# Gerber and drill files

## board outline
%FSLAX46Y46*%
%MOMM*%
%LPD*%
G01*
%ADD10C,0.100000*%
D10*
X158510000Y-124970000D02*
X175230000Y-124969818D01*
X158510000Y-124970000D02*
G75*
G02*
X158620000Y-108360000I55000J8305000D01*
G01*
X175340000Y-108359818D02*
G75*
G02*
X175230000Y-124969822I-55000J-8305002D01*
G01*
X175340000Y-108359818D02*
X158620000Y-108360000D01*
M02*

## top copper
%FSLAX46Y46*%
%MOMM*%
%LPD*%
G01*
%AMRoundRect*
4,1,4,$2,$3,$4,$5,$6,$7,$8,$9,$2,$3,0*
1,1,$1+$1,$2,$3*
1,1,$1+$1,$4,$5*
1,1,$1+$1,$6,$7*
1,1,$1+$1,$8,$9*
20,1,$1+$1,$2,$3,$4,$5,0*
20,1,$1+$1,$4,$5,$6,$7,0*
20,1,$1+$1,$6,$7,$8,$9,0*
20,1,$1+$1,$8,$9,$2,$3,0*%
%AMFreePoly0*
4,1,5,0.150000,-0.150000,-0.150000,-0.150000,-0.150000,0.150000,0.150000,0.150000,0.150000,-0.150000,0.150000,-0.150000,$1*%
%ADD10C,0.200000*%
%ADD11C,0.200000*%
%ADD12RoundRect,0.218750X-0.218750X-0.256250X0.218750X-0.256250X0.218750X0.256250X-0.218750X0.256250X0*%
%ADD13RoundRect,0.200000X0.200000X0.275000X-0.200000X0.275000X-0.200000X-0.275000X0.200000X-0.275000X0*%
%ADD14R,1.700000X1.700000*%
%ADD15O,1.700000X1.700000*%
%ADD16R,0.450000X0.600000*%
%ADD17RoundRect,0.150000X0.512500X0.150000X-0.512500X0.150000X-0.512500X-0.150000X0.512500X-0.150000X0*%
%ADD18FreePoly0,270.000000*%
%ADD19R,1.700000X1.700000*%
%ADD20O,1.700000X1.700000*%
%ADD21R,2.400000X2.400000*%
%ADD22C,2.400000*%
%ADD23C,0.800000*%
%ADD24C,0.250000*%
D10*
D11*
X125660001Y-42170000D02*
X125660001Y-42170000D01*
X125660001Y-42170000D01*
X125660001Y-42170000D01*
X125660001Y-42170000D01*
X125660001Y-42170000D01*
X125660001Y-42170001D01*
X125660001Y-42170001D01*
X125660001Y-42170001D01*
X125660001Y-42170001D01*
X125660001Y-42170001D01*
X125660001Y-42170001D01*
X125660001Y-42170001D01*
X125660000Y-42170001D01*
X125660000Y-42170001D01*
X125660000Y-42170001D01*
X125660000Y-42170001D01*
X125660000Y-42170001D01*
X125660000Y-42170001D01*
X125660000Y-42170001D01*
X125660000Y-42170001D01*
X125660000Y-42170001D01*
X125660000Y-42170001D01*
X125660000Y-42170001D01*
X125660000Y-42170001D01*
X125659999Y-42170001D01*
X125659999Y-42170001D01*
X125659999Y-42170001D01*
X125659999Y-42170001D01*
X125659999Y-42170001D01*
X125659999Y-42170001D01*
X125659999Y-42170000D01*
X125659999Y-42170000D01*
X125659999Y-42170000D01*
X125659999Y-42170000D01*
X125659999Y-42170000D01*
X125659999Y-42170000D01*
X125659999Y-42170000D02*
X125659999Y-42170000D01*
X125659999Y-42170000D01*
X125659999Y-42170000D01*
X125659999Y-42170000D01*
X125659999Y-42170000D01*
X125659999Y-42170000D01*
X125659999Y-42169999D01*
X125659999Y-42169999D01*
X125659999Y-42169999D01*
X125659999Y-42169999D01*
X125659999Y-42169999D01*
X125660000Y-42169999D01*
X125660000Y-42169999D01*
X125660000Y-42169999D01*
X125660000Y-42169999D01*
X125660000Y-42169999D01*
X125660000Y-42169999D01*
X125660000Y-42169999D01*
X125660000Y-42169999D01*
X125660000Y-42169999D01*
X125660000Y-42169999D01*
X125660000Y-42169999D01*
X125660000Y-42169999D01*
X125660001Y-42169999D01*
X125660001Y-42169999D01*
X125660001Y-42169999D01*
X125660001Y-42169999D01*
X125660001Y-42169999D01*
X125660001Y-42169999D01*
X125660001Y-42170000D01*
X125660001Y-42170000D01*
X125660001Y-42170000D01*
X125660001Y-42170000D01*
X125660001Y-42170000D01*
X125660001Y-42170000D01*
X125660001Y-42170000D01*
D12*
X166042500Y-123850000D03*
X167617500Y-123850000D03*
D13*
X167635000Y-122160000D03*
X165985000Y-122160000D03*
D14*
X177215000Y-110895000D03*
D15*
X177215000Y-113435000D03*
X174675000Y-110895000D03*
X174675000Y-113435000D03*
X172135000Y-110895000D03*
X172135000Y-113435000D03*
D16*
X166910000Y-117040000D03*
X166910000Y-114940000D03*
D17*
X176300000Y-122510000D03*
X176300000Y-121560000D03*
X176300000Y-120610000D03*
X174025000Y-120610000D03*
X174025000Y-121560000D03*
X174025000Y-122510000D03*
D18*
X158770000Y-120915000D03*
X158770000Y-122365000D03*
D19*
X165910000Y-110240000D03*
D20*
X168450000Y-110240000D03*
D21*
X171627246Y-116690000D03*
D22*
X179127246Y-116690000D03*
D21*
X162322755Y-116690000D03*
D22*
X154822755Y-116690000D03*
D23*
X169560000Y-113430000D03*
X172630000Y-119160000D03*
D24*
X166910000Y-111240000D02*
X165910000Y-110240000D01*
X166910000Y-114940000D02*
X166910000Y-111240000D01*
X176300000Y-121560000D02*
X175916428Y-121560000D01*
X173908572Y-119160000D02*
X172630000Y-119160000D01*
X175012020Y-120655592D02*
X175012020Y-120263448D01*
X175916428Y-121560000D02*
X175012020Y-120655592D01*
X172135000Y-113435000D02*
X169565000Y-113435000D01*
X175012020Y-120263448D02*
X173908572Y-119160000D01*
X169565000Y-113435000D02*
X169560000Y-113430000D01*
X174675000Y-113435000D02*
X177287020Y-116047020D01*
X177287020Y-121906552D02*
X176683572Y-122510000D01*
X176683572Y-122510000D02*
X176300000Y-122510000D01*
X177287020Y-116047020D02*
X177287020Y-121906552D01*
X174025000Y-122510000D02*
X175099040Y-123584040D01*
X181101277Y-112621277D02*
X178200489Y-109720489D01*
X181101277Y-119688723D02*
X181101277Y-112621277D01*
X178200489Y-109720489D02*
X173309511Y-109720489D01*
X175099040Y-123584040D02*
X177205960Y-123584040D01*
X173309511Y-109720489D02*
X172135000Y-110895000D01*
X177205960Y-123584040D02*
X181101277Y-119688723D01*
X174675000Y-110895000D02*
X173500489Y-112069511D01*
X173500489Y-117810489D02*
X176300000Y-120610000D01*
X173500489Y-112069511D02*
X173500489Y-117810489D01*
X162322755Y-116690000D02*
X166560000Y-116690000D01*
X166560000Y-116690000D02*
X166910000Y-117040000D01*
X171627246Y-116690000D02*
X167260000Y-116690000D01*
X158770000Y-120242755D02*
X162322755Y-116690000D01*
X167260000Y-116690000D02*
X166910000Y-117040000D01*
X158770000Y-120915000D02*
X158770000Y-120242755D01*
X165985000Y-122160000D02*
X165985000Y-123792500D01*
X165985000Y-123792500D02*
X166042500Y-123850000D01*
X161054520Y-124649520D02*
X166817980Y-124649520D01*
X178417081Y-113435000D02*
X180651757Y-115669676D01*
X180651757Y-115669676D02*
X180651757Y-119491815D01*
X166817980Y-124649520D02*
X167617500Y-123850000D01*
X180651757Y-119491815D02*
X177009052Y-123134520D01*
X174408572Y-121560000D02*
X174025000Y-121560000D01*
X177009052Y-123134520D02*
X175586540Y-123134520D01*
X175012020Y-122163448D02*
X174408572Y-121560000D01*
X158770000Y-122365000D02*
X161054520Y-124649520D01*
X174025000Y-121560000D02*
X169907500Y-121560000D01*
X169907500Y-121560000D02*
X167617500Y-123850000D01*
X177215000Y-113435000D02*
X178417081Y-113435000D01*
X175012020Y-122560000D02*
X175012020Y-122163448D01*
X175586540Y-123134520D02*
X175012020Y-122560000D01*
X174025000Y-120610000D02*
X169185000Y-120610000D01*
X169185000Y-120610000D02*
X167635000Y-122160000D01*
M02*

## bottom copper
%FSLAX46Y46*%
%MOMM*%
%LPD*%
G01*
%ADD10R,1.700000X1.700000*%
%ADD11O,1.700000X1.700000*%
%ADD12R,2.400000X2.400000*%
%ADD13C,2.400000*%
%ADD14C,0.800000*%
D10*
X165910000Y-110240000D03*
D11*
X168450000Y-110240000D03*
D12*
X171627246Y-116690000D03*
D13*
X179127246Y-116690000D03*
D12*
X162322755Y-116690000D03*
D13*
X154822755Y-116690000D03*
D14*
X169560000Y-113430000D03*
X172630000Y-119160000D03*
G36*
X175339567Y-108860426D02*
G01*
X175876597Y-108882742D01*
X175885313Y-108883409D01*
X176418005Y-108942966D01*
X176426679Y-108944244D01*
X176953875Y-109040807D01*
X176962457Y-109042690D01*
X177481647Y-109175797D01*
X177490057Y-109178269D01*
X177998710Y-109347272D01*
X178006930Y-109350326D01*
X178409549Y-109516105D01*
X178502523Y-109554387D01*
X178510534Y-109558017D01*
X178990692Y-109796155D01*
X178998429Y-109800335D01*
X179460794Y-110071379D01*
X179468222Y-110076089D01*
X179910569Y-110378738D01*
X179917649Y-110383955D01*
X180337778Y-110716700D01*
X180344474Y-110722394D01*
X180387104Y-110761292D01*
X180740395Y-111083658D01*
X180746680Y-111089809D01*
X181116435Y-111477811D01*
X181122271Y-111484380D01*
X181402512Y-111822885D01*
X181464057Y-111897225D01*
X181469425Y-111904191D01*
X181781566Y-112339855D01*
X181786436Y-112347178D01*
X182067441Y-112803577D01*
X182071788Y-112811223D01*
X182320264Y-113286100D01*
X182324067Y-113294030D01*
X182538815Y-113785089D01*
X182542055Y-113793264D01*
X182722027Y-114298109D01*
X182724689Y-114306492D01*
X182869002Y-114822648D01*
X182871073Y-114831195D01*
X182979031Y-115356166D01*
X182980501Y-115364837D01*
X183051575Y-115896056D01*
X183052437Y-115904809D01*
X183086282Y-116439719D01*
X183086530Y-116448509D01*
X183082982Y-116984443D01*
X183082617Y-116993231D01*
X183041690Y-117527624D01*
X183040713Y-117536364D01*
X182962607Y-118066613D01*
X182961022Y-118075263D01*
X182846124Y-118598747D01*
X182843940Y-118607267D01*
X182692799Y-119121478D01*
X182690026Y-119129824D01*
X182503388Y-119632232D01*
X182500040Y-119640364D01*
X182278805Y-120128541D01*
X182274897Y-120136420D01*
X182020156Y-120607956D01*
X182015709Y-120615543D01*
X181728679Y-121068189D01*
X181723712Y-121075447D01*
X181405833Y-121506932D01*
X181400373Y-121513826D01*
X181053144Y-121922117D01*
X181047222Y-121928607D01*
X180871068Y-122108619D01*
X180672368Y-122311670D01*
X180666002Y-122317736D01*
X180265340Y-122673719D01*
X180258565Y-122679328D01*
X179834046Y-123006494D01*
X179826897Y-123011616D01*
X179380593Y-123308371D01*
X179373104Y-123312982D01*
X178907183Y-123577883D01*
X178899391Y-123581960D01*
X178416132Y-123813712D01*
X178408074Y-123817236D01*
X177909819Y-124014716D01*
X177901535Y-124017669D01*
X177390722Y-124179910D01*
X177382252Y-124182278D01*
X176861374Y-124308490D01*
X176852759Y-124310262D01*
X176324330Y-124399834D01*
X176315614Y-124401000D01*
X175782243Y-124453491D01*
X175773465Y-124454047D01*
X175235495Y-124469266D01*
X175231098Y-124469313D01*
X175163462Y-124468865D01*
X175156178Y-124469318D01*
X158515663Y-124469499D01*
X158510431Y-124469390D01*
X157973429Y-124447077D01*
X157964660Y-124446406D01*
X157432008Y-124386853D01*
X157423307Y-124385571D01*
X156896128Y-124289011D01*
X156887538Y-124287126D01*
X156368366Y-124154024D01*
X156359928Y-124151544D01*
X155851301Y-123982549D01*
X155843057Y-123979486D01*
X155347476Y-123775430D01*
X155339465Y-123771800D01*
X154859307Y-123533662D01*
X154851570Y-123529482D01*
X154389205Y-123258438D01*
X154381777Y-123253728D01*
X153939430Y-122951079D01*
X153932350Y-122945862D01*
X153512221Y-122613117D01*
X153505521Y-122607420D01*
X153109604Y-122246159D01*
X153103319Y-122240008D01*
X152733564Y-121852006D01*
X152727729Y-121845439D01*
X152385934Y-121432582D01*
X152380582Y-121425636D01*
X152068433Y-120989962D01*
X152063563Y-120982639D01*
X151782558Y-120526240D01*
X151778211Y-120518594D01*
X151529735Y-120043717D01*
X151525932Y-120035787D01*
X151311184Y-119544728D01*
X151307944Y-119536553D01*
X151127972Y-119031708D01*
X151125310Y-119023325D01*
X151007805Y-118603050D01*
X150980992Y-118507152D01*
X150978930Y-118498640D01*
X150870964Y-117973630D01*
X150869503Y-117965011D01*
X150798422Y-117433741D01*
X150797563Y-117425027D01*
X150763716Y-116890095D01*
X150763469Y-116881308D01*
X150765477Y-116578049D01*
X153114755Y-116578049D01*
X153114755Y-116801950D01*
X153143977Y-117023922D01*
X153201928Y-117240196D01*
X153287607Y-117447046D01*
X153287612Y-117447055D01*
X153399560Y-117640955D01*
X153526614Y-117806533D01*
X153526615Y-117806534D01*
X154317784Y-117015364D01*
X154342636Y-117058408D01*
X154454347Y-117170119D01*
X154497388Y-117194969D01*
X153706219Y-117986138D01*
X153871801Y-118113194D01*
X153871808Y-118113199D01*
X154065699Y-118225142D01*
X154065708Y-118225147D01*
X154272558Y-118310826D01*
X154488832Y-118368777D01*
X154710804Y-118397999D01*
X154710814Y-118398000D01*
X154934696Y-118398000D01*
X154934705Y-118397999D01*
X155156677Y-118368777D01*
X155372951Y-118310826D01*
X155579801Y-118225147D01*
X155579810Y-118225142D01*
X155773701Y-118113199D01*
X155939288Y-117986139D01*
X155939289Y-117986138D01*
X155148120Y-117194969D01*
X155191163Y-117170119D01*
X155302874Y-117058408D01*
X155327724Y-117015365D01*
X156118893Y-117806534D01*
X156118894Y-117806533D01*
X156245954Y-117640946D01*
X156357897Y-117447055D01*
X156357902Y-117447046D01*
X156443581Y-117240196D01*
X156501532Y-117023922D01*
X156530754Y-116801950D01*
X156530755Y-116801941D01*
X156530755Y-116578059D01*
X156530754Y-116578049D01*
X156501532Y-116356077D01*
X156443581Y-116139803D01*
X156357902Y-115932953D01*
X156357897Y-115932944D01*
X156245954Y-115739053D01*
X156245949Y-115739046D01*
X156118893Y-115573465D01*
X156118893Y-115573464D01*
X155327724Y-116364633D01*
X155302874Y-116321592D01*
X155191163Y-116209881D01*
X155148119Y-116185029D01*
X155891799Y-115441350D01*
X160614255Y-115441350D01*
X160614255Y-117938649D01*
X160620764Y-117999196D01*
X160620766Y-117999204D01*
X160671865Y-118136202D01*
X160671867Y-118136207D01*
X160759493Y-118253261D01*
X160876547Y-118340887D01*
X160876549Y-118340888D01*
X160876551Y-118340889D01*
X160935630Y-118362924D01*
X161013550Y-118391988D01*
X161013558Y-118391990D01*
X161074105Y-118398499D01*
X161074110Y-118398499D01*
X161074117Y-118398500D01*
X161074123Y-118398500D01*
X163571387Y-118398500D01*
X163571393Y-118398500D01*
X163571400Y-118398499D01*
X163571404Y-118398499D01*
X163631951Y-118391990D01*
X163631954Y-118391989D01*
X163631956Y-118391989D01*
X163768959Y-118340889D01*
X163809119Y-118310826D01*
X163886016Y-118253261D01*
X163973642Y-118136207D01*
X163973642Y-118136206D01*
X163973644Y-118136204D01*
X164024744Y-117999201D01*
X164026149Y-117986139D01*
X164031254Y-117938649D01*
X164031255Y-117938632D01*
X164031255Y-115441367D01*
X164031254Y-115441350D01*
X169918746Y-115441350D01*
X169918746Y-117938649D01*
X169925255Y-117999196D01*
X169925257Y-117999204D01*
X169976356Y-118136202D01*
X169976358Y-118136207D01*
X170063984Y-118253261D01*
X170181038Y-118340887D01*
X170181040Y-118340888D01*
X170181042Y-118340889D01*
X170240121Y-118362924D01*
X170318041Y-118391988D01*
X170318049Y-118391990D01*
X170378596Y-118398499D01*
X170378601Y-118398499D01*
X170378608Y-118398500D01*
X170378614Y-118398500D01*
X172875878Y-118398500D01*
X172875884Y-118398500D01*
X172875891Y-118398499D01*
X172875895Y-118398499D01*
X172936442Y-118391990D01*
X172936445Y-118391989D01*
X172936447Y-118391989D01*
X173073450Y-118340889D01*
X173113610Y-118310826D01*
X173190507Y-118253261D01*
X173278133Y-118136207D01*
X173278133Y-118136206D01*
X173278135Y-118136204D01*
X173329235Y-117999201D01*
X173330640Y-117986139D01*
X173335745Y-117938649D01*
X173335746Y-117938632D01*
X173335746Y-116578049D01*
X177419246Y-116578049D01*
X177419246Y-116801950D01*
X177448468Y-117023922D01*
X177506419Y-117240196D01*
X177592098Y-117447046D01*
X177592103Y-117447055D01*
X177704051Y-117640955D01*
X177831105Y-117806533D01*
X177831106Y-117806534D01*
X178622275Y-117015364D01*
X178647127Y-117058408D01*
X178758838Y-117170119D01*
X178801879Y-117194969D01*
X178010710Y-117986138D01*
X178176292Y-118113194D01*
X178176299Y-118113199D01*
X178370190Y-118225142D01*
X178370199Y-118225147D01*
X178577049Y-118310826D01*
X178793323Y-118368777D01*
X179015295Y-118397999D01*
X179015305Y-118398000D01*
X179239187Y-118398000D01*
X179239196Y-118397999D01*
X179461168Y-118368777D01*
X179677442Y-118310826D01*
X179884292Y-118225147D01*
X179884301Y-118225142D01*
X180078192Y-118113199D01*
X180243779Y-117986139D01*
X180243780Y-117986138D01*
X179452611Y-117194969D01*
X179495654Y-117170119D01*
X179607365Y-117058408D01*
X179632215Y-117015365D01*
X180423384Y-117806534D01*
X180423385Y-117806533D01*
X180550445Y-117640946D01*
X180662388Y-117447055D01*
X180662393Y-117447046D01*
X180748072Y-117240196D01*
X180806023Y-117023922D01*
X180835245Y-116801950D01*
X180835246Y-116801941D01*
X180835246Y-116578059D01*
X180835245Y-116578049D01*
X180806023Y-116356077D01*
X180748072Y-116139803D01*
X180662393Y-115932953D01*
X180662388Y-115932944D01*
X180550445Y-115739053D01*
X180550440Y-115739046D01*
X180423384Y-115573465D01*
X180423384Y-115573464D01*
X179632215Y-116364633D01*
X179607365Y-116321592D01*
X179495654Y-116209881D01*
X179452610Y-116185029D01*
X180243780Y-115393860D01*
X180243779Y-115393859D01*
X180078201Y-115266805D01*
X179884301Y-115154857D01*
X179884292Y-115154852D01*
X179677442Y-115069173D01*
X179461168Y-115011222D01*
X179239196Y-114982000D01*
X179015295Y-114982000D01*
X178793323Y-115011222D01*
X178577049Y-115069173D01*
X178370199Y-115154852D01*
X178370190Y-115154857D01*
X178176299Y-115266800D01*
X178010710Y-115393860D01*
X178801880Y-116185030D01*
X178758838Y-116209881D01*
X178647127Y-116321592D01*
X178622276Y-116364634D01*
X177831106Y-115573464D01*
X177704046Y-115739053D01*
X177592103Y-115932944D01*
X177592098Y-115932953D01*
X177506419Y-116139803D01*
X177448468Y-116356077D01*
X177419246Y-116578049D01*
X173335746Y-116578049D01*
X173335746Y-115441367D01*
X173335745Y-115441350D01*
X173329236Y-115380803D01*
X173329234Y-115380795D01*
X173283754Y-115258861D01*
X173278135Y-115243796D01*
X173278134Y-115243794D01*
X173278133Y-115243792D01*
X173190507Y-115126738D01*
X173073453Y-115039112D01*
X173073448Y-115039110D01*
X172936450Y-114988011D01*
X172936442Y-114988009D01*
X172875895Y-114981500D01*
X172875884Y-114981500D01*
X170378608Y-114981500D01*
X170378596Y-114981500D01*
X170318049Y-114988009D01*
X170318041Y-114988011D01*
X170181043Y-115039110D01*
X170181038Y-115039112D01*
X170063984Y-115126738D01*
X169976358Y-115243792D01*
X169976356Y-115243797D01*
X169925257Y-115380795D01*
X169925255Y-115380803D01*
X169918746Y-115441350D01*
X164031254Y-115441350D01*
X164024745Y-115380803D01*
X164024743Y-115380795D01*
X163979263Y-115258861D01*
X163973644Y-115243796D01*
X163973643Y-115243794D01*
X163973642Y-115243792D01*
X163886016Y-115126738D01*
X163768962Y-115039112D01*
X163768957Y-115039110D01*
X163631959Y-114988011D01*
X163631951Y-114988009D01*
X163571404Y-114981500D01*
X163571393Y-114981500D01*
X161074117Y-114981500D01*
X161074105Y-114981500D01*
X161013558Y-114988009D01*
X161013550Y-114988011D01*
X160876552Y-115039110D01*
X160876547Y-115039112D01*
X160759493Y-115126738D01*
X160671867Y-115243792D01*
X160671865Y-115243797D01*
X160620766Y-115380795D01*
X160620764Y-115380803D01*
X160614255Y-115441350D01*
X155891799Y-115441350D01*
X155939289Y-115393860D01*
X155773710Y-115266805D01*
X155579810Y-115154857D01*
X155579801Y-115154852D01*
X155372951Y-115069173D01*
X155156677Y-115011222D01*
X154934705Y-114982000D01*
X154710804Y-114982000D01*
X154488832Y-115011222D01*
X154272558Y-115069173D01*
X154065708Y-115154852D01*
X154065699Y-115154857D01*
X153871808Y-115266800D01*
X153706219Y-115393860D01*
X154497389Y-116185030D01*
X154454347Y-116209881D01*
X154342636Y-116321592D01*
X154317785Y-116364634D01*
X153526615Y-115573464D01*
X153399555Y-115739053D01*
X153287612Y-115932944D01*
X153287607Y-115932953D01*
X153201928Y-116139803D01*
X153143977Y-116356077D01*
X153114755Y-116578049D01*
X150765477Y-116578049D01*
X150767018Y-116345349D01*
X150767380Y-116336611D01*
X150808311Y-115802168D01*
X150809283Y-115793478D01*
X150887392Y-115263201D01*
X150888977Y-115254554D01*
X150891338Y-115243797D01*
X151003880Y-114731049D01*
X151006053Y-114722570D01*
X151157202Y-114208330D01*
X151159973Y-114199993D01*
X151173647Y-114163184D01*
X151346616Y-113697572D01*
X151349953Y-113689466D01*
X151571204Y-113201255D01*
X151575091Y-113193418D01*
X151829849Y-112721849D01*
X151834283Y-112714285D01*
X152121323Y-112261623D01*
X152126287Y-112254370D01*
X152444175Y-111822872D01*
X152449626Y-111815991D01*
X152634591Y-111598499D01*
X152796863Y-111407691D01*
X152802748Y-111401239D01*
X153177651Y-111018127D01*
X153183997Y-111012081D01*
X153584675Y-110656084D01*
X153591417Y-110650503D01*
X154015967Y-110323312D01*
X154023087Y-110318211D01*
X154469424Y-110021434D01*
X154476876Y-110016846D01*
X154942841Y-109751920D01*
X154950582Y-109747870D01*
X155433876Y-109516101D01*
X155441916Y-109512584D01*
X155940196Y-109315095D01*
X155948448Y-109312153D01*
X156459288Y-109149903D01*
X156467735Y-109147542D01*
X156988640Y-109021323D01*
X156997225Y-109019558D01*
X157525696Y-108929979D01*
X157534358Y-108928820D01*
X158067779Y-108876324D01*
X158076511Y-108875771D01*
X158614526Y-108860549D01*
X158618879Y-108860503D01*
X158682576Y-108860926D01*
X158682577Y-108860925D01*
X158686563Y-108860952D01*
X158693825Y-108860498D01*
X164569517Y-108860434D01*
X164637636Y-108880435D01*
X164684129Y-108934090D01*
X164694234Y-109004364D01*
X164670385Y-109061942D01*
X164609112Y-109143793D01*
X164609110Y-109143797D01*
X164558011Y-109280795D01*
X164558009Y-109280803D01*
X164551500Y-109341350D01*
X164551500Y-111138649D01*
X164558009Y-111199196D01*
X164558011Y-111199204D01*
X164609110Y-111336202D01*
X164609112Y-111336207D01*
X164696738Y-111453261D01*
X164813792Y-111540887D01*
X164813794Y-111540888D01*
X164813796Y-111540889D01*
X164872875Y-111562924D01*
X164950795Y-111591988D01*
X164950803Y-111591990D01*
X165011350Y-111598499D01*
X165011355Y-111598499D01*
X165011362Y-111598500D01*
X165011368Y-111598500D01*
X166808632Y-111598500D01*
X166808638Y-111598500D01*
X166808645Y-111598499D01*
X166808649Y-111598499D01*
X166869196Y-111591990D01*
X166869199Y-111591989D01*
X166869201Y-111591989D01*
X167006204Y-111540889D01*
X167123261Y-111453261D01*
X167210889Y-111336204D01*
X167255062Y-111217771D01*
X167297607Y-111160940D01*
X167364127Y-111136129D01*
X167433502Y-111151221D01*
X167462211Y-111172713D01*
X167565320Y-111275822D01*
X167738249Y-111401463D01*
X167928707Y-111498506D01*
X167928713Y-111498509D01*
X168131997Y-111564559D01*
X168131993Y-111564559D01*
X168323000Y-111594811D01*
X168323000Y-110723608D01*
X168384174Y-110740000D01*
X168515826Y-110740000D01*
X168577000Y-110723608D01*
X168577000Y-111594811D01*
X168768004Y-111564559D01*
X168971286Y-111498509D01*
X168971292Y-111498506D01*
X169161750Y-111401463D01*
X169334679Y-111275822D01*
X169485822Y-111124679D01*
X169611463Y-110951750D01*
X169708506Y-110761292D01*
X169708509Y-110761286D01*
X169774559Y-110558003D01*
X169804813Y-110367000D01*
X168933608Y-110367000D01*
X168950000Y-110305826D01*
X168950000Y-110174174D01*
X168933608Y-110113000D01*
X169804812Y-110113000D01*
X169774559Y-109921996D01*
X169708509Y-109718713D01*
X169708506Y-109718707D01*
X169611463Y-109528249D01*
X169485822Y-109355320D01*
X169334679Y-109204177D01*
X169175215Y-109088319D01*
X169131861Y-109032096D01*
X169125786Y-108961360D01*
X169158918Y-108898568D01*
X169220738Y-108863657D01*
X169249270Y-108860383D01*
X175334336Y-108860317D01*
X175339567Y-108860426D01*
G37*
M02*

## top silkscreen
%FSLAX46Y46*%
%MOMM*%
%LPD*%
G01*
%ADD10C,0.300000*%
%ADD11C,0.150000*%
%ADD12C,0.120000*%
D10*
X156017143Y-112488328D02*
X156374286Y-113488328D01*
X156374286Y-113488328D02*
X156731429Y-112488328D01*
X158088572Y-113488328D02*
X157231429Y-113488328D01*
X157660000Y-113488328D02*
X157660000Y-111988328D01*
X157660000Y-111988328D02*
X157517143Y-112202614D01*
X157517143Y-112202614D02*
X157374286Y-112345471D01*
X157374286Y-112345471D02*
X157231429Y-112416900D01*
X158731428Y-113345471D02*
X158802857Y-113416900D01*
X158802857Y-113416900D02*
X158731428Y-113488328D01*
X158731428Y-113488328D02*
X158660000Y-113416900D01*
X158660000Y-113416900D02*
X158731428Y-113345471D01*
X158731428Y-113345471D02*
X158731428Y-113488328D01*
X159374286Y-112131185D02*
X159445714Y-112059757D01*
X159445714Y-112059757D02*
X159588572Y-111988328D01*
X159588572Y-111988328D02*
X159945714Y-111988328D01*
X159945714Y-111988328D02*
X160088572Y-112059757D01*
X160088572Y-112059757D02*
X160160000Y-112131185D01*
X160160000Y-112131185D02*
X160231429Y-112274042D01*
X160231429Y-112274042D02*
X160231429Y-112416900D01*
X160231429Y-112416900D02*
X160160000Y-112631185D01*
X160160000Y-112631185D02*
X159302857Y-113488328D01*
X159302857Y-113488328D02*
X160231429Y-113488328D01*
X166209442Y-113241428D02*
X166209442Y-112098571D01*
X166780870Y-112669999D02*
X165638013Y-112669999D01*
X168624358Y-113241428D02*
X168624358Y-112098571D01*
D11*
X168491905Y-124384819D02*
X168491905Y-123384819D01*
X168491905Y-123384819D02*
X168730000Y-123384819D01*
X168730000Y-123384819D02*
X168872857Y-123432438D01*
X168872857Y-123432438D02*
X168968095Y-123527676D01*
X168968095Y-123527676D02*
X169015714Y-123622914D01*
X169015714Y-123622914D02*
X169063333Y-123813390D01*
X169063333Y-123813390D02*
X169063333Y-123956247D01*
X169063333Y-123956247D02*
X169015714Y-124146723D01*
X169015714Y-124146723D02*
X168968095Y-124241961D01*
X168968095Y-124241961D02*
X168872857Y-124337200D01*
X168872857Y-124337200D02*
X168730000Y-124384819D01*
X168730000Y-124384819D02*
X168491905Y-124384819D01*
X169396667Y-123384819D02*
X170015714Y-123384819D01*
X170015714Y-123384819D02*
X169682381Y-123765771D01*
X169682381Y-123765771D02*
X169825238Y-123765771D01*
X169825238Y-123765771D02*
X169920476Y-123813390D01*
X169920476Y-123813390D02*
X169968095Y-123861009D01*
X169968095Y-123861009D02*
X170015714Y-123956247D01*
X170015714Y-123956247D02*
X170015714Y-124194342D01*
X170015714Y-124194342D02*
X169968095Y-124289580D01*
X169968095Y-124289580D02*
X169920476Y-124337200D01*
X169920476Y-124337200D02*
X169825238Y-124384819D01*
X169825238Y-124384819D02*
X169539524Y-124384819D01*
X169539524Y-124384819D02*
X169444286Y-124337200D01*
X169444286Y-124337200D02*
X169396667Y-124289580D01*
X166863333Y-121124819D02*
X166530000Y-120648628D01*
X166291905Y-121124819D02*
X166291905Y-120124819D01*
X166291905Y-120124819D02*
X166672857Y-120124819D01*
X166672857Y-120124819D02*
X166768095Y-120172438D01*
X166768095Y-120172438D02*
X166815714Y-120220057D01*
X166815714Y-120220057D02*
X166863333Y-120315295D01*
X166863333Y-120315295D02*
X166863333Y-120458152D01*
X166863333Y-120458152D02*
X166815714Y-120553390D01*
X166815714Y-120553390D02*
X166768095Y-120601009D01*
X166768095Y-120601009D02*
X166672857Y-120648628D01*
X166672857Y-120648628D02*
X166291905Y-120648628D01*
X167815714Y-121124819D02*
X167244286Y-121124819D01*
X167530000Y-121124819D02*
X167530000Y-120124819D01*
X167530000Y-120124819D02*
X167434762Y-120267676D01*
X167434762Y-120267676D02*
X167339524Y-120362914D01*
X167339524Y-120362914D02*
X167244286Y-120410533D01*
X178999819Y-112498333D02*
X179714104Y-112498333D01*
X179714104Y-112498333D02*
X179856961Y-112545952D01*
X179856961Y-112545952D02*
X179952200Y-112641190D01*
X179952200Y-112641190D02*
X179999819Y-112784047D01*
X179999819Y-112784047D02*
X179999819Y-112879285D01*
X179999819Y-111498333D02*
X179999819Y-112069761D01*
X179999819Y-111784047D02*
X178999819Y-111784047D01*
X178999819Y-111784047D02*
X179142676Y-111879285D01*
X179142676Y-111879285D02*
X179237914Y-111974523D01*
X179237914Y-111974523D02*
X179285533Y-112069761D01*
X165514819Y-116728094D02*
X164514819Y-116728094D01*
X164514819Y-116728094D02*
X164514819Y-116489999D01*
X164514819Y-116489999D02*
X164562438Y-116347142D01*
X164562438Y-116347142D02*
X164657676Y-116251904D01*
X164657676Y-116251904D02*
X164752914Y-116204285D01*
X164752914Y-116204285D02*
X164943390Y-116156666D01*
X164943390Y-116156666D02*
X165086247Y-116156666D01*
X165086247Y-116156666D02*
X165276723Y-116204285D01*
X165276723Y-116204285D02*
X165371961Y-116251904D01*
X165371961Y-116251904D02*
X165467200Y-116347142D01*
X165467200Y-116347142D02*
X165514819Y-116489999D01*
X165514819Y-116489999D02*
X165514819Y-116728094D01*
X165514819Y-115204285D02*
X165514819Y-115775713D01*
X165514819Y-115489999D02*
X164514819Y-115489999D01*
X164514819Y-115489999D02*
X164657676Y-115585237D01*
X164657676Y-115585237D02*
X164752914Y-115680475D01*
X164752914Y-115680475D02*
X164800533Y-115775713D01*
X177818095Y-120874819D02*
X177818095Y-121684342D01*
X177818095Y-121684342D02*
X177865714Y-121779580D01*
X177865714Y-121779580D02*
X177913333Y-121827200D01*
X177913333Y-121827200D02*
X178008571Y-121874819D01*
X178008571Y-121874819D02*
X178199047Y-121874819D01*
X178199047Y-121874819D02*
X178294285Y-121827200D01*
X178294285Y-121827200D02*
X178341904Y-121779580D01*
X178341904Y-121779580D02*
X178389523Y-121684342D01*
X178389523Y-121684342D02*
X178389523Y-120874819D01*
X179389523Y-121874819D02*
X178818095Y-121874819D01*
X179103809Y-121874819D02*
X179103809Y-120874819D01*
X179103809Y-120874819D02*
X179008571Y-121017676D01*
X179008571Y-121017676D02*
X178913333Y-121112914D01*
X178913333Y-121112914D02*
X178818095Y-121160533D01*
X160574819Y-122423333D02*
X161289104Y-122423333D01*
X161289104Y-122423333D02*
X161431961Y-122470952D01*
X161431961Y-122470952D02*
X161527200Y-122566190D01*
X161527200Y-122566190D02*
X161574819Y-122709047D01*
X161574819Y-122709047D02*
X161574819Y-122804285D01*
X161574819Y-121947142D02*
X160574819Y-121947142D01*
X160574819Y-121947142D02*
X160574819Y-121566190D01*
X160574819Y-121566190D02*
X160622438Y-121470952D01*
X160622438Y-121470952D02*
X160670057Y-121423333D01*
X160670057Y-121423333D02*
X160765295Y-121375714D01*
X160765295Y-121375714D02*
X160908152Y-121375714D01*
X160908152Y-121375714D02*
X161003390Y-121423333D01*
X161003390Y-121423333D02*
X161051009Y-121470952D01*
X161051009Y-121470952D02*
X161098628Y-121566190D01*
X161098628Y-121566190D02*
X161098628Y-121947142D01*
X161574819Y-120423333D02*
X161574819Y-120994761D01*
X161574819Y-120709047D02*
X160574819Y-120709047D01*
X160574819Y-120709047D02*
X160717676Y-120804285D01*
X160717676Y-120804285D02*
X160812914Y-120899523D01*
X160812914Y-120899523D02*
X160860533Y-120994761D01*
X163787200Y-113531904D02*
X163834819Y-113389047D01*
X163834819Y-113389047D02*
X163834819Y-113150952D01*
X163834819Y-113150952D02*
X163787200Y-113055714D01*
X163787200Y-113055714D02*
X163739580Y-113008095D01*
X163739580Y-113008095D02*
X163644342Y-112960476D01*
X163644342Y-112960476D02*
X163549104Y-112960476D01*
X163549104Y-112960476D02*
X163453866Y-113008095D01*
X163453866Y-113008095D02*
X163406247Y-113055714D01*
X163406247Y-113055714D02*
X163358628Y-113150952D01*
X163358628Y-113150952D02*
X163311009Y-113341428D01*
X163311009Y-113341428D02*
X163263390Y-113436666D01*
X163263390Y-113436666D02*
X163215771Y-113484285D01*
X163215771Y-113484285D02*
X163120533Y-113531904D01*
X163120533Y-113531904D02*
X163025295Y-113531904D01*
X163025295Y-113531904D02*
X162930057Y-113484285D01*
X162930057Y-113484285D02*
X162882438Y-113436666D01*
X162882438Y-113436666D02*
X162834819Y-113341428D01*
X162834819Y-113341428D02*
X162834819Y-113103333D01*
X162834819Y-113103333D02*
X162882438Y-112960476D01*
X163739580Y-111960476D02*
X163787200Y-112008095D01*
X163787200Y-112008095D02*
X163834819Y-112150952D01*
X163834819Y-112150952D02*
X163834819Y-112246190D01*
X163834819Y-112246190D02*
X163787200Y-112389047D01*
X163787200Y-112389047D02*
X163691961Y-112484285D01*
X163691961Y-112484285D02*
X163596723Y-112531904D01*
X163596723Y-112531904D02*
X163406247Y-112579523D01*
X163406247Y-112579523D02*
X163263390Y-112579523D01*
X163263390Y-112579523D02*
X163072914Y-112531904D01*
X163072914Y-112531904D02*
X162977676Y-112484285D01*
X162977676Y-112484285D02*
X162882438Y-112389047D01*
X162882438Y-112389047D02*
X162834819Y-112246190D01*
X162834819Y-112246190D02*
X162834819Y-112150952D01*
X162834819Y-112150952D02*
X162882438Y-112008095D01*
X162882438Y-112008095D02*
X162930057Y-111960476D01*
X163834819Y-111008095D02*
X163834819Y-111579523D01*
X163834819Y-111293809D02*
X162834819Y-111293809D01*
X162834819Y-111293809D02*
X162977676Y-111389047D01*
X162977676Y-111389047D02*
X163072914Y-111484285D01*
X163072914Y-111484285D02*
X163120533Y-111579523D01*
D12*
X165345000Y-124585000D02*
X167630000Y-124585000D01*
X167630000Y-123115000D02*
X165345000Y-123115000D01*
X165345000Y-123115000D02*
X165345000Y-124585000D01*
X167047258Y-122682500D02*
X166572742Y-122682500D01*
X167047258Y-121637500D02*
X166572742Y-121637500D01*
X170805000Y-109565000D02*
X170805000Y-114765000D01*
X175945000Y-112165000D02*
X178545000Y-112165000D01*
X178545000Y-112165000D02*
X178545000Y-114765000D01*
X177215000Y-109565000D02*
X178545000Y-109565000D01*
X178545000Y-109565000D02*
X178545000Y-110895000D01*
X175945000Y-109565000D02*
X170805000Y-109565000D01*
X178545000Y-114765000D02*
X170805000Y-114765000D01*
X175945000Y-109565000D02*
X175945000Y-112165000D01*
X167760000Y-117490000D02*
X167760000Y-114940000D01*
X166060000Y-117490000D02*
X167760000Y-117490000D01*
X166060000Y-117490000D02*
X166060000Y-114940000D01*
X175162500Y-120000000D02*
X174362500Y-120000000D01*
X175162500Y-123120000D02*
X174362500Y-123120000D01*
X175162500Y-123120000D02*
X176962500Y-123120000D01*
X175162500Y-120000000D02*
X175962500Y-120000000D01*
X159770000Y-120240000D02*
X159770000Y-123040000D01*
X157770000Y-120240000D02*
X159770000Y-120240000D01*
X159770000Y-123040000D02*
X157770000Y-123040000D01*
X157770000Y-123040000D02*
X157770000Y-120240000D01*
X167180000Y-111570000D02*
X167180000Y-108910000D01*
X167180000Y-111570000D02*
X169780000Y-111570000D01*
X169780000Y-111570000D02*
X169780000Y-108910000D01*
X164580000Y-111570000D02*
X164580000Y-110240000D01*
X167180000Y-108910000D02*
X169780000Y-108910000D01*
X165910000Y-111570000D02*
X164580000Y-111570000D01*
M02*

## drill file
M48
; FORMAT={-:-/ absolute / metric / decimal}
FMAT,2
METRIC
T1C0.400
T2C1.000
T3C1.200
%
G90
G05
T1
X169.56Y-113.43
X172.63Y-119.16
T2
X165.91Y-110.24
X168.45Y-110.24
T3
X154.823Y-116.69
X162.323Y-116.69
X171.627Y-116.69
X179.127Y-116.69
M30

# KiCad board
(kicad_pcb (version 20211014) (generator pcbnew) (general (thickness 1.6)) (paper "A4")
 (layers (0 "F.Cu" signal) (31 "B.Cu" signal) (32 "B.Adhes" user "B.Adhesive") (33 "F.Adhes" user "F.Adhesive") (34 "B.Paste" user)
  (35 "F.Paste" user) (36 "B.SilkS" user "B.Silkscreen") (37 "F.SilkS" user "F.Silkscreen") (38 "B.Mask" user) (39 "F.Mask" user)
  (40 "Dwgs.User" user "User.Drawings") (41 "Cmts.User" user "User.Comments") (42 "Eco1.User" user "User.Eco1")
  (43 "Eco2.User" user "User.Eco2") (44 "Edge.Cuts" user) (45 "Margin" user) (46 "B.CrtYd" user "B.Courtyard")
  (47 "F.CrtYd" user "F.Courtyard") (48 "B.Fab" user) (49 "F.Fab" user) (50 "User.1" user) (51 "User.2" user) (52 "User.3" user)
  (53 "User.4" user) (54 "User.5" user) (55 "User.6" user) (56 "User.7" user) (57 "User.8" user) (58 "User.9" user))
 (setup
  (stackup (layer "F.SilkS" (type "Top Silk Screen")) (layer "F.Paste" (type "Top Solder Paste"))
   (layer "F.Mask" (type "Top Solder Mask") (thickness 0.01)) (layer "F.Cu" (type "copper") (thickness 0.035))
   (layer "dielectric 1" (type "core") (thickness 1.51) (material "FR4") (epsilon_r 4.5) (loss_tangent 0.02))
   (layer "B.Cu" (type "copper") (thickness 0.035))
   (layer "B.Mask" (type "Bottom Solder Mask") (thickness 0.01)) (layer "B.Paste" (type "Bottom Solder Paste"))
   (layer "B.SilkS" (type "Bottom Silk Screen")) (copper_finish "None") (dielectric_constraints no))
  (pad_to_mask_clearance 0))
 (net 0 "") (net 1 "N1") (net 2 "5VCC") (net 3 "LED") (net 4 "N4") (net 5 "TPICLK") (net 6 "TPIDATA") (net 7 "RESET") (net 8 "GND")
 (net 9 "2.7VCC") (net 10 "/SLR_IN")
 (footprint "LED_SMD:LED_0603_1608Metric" (layer "F.Cu") (at 166.83 123.85)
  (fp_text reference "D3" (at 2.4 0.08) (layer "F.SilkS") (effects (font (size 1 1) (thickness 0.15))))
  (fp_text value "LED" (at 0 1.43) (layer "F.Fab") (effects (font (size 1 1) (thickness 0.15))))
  (fp_line (start -1.485 0.735) (end 0.8 0.735) (layer "F.SilkS") (width 0.12))
  (fp_line (start 0.8 -0.735) (end -1.485 -0.735) (layer "F.SilkS") (width 0.12))
  (fp_line (start -1.485 -0.735) (end -1.485 0.735) (layer "F.SilkS") (width 0.12))
  (pad "1" smd roundrect (at -0.7875 0) (size 0.875 0.95) (layers "F.Cu" "F.Paste" "F.Mask") (roundrect_rratio 0.25) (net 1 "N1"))
  (pad "2" smd roundrect (at 0.7875 0) (size 0.875 0.95) (layers "F.Cu" "F.Paste" "F.Mask") (roundrect_rratio 0.25) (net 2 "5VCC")))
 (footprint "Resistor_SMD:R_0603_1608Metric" (layer "F.Cu") (at 166.81 122.16 180)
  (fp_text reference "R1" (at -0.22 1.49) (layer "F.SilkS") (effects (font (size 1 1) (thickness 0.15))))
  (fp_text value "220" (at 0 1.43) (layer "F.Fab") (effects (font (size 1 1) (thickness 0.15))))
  (fp_line (start -0.237258 -0.5225) (end 0.237258 -0.5225) (layer "F.SilkS") (width 0.12))
  (fp_line (start -0.237258 0.5225) (end 0.237258 0.5225) (layer "F.SilkS") (width 0.12))
  (pad "1" smd roundrect (at -0.825 0 180) (size 0.8 0.95) (layers "F.Cu" "F.Paste" "F.Mask") (roundrect_rratio 0.25) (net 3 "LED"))
  (pad "2" smd roundrect (at 0.825 0 180) (size 0.8 0.95) (layers "F.Cu" "F.Paste" "F.Mask") (roundrect_rratio 0.25) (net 1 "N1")))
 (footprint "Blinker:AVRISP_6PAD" (layer "F.Cu") (at 177.215 110.895 -90)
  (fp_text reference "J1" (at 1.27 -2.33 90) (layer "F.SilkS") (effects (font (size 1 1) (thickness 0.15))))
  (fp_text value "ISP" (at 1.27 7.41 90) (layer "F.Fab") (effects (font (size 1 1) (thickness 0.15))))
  (fp_line (start -1.33 6.41) (end 3.87 6.41) (layer "F.SilkS") (width 0.12))
  (fp_line (start 1.27 1.27) (end 1.27 -1.33) (layer "F.SilkS") (width 0.12))
  (fp_line (start 1.27 -1.33) (end 3.87 -1.33) (layer "F.SilkS") (width 0.12))
  (fp_line (start -1.33 0) (end -1.33 -1.33) (layer "F.SilkS") (width 0.12))
  (fp_line (start -1.33 -1.33) (end 0 -1.33) (layer "F.SilkS") (width 0.12))
  (fp_line (start -1.33 1.27) (end -1.33 6.41) (layer "F.SilkS") (width 0.12))
  (fp_line (start 3.87 -1.33) (end 3.87 6.41) (layer "F.SilkS") (width 0.12))
  (fp_line (start -1.33 1.27) (end 1.27 1.27) (layer "F.SilkS") (width 0.12))
  (pad "1" smd rect (at 0 0 270) (size 1.7 1.7) (layers "F.Cu" "F.Mask") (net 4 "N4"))
  (pad "2" smd oval (at 2.54 0 270) (size 1.7 1.7) (layers "F.Cu" "F.Mask") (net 2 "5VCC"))
  (pad "3" smd oval (at 0 2.54 270) (size 1.7 1.7) (layers "F.Cu" "F.Mask") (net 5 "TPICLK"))
  (pad "4" smd oval (at 2.54 2.54 270) (size 1.7 1.7) (layers "F.Cu" "F.Mask") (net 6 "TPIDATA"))
  (pad "5" smd oval (at 0 5.08 270) (size 1.7 1.7) (layers "F.Cu" "F.Mask") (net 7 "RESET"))
  (pad "6" smd oval (at 2.54 5.08 270) (size 1.7 1.7) (layers "F.Cu" "F.Mask") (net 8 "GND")))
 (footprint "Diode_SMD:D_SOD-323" (layer "F.Cu") (at 166.91 115.99 90)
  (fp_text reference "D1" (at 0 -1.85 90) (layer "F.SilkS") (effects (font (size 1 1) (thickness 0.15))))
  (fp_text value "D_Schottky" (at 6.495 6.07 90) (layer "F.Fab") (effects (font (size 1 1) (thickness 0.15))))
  (fp_line (start -1.5 0.85) (end 1.05 0.85) (layer "F.SilkS") (width 0.12))
  (fp_line (start -1.5 -0.85) (end -1.5 0.85) (layer "F.SilkS") (width 0.12))
  (fp_line (start -1.5 -0.85) (end 1.05 -0.85) (layer "F.SilkS") (width 0.12))
  (pad "1" smd rect (at -1.05 0 90) (size 0.6 0.45) (layers "F.Cu" "F.Paste" "F.Mask") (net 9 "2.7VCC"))
  (pad "2" smd rect (at 1.05 0 90) (size 0.6 0.45) (layers "F.Cu" "F.Paste" "F.Mask") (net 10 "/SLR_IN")))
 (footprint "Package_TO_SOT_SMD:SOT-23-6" (layer "F.Cu") (at 175.1625 121.56 180)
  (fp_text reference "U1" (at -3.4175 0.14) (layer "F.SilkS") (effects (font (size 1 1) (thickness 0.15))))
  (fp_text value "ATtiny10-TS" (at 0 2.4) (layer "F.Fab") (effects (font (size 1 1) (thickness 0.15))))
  (fp_line (start 0 1.56) (end 0.8 1.56) (layer "F.SilkS") (width 0.12))
  (fp_line (start 0 -1.56) (end 0.8 -1.56) (layer "F.SilkS") (width 0.12))
  (fp_line (start 0 -1.56) (end -1.8 -1.56) (layer "F.SilkS") (width 0.12))
  (fp_line (start 0 1.56) (end -0.8 1.56) (layer "F.SilkS") (width 0.12))
  (pad "1" smd roundrect (at -1.1375 -0.95 180) (size 1.325 0.6) (layers "F.Cu" "F.Paste" "F.Mask") (roundrect_rratio 0.25)
   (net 6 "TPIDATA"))
  (pad "2" smd roundrect (at -1.1375 0 180) (size 1.325 0.6) (layers "F.Cu" "F.Paste" "F.Mask") (roundrect_rratio 0.25) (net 8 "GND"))
  (pad "3" smd roundrect (at -1.1375 0.95 180) (size 1.325 0.6) (layers "F.Cu" "F.Paste" "F.Mask") (roundrect_rratio 0.25) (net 5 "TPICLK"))
  (pad "4" smd roundrect (at 1.1375 0.95 180) (size 1.325 0.6) (layers "F.Cu" "F.Paste" "F.Mask") (roundrect_rratio 0.25) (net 3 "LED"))
  (pad "5" smd roundrect (at 1.1375 0 180) (size 1.325 0.6) (layers "F.Cu" "F.Paste" "F.Mask") (roundrect_rratio 0.25) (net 2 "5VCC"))
  (pad "6" smd roundrect (at 1.1375 -0.95 180) (size 1.325 0.6) (layers "F.Cu" "F.Paste" "F.Mask") (roundrect_rratio 0.25) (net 7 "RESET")))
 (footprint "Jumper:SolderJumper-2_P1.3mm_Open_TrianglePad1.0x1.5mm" (layer "F.Cu") (at 158.77 121.64 -90)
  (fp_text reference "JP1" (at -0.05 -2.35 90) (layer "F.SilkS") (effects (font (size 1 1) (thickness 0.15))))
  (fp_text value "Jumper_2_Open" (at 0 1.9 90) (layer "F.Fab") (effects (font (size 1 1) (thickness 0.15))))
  (fp_line (start -1.4 -1) (end 1.4 -1) (layer "F.SilkS") (width 0.12))
  (fp_line (start -1.4 1) (end -1.4 -1) (layer "F.SilkS") (width 0.12))
  (fp_line (start 1.4 -1) (end 1.4 1) (layer "F.SilkS") (width 0.12))
  (fp_line (start 1.4 1) (end -1.4 1) (layer "F.SilkS") (width 0.12))
  (pad "1" smd custom (at -0.725 0 270) (size 0.3 0.3) (layers "F.Cu" "F.Mask") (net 9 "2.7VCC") (zone_connect 2)
   (options (clearance outline) (anchor rect)) (primitives))
  (pad "2" smd custom (at 0.725 0 270) (size 0.3 0.3) (layers "F.Cu" "F.Mask") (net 2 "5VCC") (zone_connect 2)
   (options (clearance outline) (anchor rect)) (primitives)))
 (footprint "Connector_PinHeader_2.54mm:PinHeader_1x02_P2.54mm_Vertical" (layer "F.Cu") (at 165.91 110.24 90)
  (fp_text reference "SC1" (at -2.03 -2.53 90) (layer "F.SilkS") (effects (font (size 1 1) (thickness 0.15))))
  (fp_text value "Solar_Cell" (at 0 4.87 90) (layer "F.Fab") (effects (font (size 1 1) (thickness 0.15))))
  (fp_line (start -1.33 1.27) (end 1.33 1.27) (layer "F.SilkS") (width 0.12))
  (fp_line (start -1.33 1.27) (end -1.33 3.87) (layer "F.SilkS") (width 0.12))
  (fp_line (start -1.33 3.87) (end 1.33 3.87) (layer "F.SilkS") (width 0.12))
  (fp_line (start -1.33 -1.33) (end 0 -1.33) (layer "F.SilkS") (width 0.12))
  (fp_line (start 1.33 1.27) (end 1.33 3.87) (layer "F.SilkS") (width 0.12))
  (fp_line (start -1.33 0) (end -1.33 -1.33) (layer "F.SilkS") (width 0.12))
  (pad "1" thru_hole rect (at 0 0 90) (size 1.7 1.7) (drill 1) (layers *.Cu *.Mask) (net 10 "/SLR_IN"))
  (pad "2" thru_hole oval (at 0 2.54 90) (size 1.7 1.7) (drill 1) (layers *.Cu *.Mask) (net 8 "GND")))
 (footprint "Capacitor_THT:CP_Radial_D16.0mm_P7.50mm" (layer "B.Cu") (at 171.627246 116.69)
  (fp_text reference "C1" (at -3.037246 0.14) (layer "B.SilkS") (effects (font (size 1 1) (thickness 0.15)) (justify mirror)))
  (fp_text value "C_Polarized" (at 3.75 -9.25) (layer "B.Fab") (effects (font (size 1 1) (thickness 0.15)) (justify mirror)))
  (pad "1" thru_hole rect (at 0 0) (size 2.4 2.4) (drill 1.2) (layers *.Cu *.Mask) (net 9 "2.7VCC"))
  (pad "2" thru_hole circle (at 7.5 0) (size 2.4 2.4) (drill 1.2) (layers *.Cu *.Mask) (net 8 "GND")))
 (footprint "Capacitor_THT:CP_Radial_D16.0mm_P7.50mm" (layer "B.Cu") (at 162.322755 116.69 180)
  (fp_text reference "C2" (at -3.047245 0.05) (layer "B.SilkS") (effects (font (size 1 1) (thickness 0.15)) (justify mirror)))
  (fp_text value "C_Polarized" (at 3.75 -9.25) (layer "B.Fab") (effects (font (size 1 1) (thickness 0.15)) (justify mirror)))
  (pad "1" thru_hole rect (at 0 0 180) (size 2.4 2.4) (drill 1.2) (layers *.Cu *.Mask) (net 9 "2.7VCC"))
  (pad "2" thru_hole circle (at 7.5 0 180) (size 2.4 2.4) (drill 1.2) (layers *.Cu *.Mask) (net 8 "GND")))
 (gr_circle (center 125.66 42.17) (end 125.66 42.17) (layer "F.Cu") (width 0.2) (fill none))
 (gr_line (start 158.51 124.97) (end 175.23 124.969818) (layer "Edge.Cuts") (width 0.1))
 (gr_arc (start 158.51 124.97) (mid 150.26 116.61) (end 158.62 108.36) (layer "Edge.Cuts") (width 0.1))
 (gr_arc (start 175.34 108.359818) (mid 183.59 116.719818) (end 175.23 124.969818) (layer "Edge.Cuts") (width 0.1))
 (gr_line (start 175.34 108.359818) (end 158.62 108.36) (layer "Edge.Cuts") (width 0.1))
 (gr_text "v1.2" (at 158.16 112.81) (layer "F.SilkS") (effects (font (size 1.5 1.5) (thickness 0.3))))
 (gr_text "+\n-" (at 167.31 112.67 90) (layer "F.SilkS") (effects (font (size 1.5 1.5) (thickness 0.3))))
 (segment (start 166.91 111.24) (end 165.91 110.24) (width 0.25) (layer "F.Cu") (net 10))
 (segment (start 166.91 114.94) (end 166.91 111.24) (width 0.25) (layer "F.Cu") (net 10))
 (segment (start 176.3 121.56) (end 175.916428 121.56) (width 0.25) (layer "F.Cu") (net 8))
 (segment (start 173.908572 119.16) (end 172.63 119.16) (width 0.25) (layer "F.Cu") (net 8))
 (segment (start 175.01202 120.655592) (end 175.01202 120.263448) (width 0.25) (layer "F.Cu") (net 8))
 (segment (start 175.916428 121.56) (end 175.01202 120.655592) (width 0.25) (layer "F.Cu") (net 8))
 (segment (start 172.135 113.435) (end 169.565 113.435) (width 0.25) (layer "F.Cu") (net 8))
 (segment (start 175.01202 120.263448) (end 173.908572 119.16) (width 0.25) (layer "F.Cu") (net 8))
 (segment (start 169.565 113.435) (end 169.56 113.43) (width 0.25) (layer "F.Cu") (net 8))
 (via (at 169.56 113.43) (size 0.8) (drill 0.4) (layers "F.Cu" "B.Cu") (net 8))
 (via (at 172.63 119.16) (size 0.8) (drill 0.4) (layers "F.Cu" "B.Cu") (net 8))
 (segment (start 174.675 113.435) (end 177.28702 116.04702) (width 0.25) (layer "F.Cu") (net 6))
 (segment (start 177.28702 121.906552) (end 176.683572 122.51) (width 0.25) (layer "F.Cu") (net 6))
 (segment (start 176.683572 122.51) (end 176.3 122.51) (width 0.25) (layer "F.Cu") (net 6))
 (segment (start 177.28702 116.04702) (end 177.28702 121.906552) (width 0.25) (layer "F.Cu") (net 6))
 (segment (start 174.025 122.51) (end 175.09904 123.58404) (width 0.25) (layer "F.Cu") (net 7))
 (segment (start 181.101277 112.621277) (end 178.200489 109.720489) (width 0.25) (layer "F.Cu") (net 7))
 (segment (start 181.101277 119.688723) (end 181.101277 112.621277) (width 0.25) (layer "F.Cu") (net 7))
 (segment (start 178.200489 109.720489) (end 173.309511 109.720489) (width 0.25) (layer "F.Cu") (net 7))
 (segment (start 175.09904 123.58404) (end 177.20596 123.58404) (width 0.25) (layer "F.Cu") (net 7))
 (segment (start 173.309511 109.720489) (end 172.135 110.895) (width 0.25) (layer "F.Cu") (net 7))
 (segment (start 177.20596 123.58404) (end 181.101277 119.688723) (width 0.25) (layer "F.Cu") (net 7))
 (segment (start 174.675 110.895) (end 173.500489 112.069511) (width 0.25) (layer "F.Cu") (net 5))
 (segment (start 173.500489 117.810489) (end 176.3 120.61) (width 0.25) (layer "F.Cu") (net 5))
 (segment (start 173.500489 112.069511) (end 173.500489 117.810489) (width 0.25) (layer "F.Cu") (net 5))
 (segment (start 162.322755 116.69) (end 166.56 116.69) (width 0.25) (layer "F.Cu") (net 9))
 (segment (start 166.56 116.69) (end 166.91 117.04) (width 0.25) (layer "F.Cu") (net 9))
 (segment (start 171.627246 116.69) (end 167.26 116.69) (width 0.25) (layer "F.Cu") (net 9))
 (segment (start 158.77 120.242755) (end 162.322755 116.69) (width 0.25) (layer "F.Cu") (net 9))
 (segment (start 167.26 116.69) (end 166.91 117.04) (width 0.25) (layer "F.Cu") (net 9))
 (segment (start 158.77 120.915) (end 158.77 120.242755) (width 0.25) (layer "F.Cu") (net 9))
 (segment (start 165.985 122.16) (end 165.985 123.7925) (width 0.25) (layer "F.Cu") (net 1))
 (segment (start 165.985 123.7925) (end 166.0425 123.85) (width 0.25) (layer "F.Cu") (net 1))
 (segment (start 161.05452 124.64952) (end 166.81798 124.64952) (width 0.25) (layer "F.Cu") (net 2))
 (segment (start 178.417081 113.435) (end 180.651757 115.669676) (width 0.25) (layer "F.Cu") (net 2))
 (segment (start 180.651757 115.669676) (end 180.651757 119.491815) (width 0.25) (layer "F.Cu") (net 2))
 (segment (start 166.81798 124.64952) (end 167.6175 123.85) (width 0.25) (layer "F.Cu") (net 2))
 (segment (start 180.651757 119.491815) (end 177.009052 123.13452) (width 0.25) (layer "F.Cu") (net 2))
 (segment (start 174.408572 121.56) (end 174.025 121.56) (width 0.25) (layer "F.Cu") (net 2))
 (segment (start 177.009052 123.13452) (end 175.58654 123.13452) (width 0.25) (layer "F.Cu") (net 2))
 (segment (start 175.01202 122.163448) (end 174.408572 121.56) (width 0.25) (layer "F.Cu") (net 2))
 (segment (start 158.77 122.365) (end 161.05452 124.64952) (width 0.25) (layer "F.Cu") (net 2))
 (segment (start 174.025 121.56) (end 169.9075 121.56) (width 0.25) (layer "F.Cu") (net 2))
 (segment (start 169.9075 121.56) (end 167.6175 123.85) (width 0.25) (layer "F.Cu") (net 2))
 (segment (start 177.215 113.435) (end 178.417081 113.435) (width 0.25) (layer "F.Cu") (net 2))
 (segment (start 175.01202 122.56) (end 175.01202 122.163448) (width 0.25) (layer "F.Cu") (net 2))
 (segment (start 175.58654 123.13452) (end 175.01202 122.56) (width 0.25) (layer "F.Cu") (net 2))
 (segment (start 174.025 120.61) (end 169.185 120.61) (width 0.25) (layer "F.Cu") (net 3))
 (segment (start 169.185 120.61) (end 167.635 122.16) (width 0.25) (layer "F.Cu") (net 3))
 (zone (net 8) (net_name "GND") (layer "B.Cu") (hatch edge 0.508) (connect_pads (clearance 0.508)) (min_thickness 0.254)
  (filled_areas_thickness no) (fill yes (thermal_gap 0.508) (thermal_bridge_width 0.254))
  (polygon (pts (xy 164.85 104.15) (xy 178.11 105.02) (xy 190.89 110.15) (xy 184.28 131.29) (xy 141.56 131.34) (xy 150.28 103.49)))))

